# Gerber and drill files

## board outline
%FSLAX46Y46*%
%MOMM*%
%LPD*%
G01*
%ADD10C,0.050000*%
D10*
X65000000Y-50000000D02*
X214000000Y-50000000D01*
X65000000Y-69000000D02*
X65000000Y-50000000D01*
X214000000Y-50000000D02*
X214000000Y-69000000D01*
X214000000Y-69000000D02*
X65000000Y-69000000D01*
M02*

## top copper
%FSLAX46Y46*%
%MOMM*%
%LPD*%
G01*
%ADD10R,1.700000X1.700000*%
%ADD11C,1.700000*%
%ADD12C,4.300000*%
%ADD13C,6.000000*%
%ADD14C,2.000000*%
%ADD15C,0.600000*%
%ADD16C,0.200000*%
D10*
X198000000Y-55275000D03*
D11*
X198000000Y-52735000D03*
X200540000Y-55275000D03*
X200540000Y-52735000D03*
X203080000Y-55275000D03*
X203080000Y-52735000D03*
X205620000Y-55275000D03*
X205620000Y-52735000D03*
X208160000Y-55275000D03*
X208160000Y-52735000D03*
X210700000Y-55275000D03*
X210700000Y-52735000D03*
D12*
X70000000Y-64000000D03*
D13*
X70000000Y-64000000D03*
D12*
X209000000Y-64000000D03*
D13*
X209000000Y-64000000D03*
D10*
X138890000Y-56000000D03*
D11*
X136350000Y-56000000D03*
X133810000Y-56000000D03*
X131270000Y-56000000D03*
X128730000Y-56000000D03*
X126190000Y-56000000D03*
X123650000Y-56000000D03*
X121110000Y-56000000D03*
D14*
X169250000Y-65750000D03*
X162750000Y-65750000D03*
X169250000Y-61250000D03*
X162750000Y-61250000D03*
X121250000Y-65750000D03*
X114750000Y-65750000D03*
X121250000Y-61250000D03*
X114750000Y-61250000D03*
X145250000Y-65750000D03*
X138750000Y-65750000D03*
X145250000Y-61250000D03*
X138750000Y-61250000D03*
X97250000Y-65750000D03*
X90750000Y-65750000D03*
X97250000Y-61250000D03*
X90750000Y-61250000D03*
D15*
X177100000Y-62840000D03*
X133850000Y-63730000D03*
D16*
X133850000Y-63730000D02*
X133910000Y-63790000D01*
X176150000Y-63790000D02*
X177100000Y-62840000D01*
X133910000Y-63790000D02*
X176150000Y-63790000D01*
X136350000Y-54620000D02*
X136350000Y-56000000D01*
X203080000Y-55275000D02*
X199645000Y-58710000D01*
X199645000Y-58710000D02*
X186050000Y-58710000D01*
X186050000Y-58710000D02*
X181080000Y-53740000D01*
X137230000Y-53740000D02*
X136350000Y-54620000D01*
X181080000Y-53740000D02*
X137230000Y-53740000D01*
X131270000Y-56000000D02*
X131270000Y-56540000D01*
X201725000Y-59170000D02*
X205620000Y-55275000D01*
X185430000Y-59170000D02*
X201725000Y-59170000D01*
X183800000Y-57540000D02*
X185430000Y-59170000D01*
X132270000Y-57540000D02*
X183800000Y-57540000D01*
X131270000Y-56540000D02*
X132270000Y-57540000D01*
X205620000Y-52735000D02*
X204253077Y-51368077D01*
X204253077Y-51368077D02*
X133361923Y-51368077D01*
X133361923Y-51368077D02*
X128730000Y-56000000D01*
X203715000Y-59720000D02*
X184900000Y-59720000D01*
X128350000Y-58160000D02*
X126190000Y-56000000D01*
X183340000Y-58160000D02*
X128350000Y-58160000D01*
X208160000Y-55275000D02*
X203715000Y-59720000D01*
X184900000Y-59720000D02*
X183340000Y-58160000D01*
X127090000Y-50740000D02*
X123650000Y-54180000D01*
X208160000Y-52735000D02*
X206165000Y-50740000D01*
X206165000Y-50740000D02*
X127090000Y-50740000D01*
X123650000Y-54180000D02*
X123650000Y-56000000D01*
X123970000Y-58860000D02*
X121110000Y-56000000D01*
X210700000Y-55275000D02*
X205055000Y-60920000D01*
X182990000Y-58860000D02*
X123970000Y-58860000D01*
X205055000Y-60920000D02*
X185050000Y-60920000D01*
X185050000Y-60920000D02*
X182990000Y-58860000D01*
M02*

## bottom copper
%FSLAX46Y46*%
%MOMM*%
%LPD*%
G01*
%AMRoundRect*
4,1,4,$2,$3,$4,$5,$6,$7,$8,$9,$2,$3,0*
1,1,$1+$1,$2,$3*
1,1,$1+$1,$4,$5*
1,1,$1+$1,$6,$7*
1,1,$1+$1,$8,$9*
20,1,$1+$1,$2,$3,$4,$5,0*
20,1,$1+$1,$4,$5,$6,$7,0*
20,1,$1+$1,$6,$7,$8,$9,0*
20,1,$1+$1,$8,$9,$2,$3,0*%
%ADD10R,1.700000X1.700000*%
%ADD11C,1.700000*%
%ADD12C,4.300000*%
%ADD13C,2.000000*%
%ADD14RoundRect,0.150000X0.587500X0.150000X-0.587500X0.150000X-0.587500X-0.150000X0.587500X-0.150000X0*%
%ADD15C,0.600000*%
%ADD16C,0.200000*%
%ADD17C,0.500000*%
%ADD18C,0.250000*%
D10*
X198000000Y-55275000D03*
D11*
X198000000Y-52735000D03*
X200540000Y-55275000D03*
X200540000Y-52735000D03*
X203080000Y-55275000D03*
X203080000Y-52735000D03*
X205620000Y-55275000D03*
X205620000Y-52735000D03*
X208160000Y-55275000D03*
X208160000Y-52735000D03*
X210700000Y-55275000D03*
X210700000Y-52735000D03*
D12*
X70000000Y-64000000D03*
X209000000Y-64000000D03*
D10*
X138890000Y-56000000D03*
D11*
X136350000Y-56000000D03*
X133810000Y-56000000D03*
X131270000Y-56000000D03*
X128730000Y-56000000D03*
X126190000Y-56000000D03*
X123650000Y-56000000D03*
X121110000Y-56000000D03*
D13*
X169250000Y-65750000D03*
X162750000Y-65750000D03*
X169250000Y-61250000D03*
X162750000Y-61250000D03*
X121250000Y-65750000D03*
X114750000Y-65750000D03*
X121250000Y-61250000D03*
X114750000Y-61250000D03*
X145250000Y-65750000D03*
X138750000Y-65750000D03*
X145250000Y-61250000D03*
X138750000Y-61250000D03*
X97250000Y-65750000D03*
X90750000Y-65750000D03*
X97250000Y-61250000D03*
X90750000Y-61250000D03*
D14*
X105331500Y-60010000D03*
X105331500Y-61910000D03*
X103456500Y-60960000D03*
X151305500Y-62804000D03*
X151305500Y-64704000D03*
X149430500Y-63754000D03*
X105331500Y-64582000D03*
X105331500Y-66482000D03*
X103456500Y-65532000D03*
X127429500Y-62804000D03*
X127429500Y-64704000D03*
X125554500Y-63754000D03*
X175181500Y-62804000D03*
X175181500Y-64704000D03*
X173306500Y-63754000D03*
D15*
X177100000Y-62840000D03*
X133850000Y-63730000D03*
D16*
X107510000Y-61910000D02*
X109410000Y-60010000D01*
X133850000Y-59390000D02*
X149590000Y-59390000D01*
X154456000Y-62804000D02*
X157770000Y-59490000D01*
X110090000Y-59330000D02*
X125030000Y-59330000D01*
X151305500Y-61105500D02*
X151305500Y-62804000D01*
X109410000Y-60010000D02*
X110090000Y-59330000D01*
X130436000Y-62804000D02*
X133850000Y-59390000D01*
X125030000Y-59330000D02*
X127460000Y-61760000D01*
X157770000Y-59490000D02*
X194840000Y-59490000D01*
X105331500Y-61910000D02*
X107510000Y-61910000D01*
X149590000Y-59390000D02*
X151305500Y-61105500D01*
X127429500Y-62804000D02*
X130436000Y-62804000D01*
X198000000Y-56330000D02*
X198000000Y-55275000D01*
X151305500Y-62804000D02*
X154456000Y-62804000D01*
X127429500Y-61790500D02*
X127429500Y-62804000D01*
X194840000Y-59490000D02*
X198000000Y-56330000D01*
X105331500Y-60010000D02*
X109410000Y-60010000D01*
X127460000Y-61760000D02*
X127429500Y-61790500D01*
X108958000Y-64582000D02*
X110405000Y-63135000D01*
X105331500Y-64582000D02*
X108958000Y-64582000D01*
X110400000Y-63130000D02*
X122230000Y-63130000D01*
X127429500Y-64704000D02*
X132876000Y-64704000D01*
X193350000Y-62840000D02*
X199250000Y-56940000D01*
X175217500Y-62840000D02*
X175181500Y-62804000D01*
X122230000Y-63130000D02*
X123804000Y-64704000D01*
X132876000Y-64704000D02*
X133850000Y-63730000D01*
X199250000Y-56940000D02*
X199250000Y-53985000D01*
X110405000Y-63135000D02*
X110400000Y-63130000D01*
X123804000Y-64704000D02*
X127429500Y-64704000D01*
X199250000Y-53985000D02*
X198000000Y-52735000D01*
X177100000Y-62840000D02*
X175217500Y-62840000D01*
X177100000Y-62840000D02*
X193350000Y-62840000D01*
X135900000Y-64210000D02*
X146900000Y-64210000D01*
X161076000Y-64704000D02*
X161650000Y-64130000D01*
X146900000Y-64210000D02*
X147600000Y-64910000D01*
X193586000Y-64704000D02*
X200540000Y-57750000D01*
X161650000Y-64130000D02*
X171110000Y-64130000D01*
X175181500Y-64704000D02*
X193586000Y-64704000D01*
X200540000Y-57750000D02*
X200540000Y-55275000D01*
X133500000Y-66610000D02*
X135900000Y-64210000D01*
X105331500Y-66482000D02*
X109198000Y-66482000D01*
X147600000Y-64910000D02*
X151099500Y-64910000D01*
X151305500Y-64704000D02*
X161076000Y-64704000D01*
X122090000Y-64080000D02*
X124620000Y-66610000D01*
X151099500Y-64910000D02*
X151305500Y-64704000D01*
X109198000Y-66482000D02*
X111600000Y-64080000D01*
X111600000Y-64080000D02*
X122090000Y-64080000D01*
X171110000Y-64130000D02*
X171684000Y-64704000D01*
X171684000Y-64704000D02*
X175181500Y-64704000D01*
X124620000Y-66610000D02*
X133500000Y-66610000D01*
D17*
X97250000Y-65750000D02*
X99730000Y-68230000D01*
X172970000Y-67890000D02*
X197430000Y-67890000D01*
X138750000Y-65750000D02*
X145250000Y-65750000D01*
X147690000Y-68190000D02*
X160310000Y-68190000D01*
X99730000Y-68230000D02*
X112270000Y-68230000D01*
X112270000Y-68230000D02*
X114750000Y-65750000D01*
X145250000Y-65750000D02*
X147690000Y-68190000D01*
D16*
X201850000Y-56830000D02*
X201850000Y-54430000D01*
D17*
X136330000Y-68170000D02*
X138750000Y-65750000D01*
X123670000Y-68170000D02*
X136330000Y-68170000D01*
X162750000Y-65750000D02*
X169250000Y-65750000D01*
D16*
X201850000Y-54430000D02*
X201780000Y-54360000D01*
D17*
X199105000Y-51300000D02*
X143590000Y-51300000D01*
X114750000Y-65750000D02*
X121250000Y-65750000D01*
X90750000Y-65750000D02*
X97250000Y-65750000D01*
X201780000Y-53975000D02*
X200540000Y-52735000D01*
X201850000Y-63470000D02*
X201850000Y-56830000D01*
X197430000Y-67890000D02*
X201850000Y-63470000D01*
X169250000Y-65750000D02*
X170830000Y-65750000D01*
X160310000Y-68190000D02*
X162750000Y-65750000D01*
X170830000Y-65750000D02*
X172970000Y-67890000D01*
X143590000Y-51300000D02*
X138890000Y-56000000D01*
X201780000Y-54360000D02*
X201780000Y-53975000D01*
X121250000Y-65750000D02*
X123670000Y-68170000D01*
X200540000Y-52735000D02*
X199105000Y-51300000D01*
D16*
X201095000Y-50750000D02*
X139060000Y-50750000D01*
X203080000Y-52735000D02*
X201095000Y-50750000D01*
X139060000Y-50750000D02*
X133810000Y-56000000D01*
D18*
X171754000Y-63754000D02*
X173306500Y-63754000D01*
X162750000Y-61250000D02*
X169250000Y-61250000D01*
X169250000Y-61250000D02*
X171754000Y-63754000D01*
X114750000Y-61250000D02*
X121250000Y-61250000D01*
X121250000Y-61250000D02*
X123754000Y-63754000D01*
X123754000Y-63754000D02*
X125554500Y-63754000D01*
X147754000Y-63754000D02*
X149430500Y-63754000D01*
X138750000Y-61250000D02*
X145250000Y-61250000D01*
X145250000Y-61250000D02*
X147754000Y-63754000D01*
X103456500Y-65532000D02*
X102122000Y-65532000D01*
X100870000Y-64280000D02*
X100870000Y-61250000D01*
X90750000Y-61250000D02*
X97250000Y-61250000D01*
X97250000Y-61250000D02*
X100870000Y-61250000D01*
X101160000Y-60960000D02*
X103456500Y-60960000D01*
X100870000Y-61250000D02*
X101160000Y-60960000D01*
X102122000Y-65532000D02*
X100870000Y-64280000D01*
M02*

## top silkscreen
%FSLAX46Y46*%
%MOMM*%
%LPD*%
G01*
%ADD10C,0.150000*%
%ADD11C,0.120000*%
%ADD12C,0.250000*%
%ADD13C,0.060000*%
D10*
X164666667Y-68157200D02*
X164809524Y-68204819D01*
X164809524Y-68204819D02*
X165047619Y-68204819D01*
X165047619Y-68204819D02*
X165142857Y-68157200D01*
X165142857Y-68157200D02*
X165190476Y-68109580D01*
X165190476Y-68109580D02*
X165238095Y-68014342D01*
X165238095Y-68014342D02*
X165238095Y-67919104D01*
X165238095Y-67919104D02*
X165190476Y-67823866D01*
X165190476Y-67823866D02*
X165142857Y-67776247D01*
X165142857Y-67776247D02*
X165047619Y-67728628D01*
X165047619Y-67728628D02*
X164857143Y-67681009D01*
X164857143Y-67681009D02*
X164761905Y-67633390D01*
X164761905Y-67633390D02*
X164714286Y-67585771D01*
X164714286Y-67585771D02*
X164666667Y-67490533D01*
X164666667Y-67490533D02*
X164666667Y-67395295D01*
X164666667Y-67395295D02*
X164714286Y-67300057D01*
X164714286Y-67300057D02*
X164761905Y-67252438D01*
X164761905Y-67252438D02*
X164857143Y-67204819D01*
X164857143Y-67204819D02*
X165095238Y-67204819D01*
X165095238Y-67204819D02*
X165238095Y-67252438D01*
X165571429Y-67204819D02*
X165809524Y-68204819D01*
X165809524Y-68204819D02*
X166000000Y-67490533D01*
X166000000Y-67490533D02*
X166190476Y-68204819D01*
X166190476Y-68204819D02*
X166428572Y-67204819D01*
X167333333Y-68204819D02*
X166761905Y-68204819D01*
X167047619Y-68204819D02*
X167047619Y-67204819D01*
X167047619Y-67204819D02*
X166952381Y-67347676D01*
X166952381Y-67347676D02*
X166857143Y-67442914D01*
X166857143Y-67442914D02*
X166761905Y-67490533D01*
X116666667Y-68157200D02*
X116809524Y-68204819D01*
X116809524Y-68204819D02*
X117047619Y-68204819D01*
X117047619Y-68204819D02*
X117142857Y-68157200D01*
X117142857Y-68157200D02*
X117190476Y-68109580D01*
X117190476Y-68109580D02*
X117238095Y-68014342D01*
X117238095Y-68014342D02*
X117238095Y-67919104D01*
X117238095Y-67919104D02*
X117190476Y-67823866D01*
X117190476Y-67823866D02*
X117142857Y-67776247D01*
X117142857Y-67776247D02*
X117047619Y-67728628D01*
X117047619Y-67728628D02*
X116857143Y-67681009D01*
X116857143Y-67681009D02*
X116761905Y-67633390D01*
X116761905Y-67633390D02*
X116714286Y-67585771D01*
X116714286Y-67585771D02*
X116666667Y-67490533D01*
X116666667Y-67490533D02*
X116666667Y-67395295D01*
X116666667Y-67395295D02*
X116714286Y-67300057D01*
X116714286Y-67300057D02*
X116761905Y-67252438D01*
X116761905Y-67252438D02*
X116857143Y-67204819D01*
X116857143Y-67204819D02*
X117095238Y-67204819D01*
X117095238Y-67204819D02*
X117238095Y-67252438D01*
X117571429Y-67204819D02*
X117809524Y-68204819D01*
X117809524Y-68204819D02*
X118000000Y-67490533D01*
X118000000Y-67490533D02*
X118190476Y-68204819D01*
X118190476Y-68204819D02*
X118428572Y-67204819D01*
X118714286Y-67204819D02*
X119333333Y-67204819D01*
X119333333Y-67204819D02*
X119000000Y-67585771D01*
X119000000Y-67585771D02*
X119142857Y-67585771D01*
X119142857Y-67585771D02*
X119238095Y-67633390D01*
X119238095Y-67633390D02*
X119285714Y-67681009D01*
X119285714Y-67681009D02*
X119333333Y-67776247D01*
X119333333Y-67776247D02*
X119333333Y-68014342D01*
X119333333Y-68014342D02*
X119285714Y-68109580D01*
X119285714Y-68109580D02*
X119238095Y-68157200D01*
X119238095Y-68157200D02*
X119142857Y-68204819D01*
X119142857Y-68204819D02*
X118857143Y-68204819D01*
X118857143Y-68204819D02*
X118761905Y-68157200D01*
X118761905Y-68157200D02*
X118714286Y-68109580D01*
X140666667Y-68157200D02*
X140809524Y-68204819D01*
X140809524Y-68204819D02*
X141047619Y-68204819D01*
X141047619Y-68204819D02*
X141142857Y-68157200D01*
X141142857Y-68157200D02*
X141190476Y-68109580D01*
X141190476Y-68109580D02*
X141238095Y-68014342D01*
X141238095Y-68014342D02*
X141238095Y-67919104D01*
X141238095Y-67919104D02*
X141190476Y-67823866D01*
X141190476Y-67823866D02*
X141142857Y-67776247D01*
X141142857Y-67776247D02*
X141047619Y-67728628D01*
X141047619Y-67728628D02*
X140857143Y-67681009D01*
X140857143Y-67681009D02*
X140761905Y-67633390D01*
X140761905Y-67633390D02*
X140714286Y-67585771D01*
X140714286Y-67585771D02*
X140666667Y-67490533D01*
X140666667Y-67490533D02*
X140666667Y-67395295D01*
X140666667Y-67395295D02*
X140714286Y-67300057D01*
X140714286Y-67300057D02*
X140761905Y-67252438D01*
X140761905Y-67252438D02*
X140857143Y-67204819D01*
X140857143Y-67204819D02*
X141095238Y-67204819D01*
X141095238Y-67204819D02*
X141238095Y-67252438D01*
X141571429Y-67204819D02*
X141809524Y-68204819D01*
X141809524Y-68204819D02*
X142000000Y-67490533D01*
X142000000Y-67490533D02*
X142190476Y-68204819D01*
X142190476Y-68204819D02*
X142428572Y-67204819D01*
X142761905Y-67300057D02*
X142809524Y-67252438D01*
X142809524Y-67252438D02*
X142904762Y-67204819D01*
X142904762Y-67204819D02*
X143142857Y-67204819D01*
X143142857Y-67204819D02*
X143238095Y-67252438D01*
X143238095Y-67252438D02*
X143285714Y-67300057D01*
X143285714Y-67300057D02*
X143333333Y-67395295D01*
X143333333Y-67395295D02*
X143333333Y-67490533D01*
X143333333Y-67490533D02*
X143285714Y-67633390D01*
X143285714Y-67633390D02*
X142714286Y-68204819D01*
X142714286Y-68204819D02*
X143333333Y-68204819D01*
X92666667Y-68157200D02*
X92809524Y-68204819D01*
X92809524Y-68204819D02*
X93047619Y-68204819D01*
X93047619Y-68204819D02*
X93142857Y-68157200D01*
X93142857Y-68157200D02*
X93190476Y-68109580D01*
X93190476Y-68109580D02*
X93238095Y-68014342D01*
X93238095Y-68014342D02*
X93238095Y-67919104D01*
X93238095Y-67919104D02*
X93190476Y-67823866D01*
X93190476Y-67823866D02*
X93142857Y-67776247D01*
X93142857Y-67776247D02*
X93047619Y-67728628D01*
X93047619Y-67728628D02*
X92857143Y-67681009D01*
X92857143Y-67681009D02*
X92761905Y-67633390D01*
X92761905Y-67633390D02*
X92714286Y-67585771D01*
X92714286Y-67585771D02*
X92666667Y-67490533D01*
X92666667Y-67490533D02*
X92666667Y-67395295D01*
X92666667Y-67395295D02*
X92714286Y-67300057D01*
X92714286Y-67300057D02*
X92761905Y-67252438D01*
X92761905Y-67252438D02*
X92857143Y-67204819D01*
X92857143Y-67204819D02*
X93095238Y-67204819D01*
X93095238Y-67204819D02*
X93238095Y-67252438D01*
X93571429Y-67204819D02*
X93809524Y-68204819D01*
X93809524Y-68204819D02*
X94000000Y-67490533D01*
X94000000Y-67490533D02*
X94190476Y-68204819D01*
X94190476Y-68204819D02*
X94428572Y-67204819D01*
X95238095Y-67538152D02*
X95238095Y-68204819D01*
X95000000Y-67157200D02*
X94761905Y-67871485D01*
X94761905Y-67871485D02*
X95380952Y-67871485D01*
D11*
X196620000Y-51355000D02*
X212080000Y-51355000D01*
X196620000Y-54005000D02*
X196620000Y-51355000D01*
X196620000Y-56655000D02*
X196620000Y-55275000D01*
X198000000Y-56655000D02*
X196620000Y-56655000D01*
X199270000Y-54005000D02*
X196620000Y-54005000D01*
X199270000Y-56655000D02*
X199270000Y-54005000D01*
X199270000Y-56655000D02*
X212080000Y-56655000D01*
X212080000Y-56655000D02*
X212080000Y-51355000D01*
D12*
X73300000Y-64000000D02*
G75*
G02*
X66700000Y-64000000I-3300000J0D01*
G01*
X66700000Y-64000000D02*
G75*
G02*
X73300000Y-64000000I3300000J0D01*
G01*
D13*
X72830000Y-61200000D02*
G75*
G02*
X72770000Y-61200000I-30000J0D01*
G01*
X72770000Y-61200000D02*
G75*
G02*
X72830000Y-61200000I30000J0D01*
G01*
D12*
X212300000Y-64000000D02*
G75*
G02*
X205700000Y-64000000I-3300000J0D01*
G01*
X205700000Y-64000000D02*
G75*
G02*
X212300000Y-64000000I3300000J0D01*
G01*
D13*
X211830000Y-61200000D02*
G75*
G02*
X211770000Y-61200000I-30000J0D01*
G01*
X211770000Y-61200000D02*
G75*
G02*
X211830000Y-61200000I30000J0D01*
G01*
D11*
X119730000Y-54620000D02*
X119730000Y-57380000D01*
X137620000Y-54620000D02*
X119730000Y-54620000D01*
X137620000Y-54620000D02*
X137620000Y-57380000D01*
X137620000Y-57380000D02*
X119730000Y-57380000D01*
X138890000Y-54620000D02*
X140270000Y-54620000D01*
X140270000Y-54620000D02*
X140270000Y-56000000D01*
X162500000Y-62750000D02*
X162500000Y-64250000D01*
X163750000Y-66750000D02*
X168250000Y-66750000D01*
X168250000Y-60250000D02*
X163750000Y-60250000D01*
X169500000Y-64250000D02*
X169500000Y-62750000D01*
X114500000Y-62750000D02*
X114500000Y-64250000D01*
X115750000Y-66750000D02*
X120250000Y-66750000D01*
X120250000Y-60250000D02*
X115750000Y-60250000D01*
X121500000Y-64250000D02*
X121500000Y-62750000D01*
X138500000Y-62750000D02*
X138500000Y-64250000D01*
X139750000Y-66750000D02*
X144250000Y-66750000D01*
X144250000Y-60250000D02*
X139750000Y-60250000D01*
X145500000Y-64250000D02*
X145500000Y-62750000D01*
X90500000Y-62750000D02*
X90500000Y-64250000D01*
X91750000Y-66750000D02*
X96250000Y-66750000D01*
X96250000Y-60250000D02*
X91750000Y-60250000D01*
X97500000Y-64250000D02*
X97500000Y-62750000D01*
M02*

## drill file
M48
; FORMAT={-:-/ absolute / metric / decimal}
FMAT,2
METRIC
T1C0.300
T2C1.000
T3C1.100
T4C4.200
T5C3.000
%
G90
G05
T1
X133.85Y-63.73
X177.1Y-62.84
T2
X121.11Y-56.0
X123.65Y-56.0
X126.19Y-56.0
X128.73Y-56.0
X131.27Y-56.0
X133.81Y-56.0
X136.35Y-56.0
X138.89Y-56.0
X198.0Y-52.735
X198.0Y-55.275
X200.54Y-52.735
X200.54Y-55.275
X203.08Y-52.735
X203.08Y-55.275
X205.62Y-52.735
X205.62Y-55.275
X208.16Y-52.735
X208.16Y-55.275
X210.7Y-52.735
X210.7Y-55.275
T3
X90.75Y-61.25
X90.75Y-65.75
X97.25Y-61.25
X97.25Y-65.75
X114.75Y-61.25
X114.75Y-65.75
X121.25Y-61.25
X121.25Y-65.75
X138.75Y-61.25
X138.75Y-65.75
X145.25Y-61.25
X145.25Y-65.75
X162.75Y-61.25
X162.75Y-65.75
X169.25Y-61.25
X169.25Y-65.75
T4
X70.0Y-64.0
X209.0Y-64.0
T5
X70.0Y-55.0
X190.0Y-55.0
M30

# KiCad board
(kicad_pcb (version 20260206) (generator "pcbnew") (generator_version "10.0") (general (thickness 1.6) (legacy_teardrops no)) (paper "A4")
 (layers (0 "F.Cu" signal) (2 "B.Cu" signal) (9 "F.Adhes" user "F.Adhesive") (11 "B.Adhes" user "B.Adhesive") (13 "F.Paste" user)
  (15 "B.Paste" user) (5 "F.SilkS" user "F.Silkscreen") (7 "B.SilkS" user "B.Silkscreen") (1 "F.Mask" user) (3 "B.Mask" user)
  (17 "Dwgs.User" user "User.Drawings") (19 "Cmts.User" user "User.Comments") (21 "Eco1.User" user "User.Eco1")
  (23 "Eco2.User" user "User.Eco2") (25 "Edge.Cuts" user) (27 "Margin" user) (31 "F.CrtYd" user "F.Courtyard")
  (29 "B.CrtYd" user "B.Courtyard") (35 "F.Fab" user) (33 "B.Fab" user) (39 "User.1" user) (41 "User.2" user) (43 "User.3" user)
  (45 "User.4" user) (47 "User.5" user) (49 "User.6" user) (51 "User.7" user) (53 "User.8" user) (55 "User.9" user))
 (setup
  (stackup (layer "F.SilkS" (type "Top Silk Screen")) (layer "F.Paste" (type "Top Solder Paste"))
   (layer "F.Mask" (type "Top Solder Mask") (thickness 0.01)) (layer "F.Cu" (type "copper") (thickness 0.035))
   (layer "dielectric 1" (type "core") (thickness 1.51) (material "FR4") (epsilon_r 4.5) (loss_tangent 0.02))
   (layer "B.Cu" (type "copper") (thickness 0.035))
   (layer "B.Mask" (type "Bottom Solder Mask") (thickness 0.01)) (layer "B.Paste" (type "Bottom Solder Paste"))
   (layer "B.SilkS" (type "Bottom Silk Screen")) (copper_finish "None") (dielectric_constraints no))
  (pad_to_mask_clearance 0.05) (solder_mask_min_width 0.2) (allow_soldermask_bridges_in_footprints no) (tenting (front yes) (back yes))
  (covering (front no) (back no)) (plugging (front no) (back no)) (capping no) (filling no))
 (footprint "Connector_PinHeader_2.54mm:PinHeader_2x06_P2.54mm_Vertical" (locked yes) (layer "F.Cu") (at 198 55.275 90)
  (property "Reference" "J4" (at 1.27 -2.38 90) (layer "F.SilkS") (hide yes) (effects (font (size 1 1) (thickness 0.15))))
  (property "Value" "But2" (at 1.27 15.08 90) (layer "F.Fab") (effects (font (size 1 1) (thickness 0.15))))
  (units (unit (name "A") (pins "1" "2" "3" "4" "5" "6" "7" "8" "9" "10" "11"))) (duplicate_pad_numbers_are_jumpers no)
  (fp_line (start 3.92 -1.38) (end 3.92 14.08) (stroke (width 0.12) (type solid)) (layer "F.SilkS"))
  (fp_line (start 1.27 -1.38) (end 3.92 -1.38) (stroke (width 0.12) (type solid)) (layer "F.SilkS"))
  (fp_line (start -1.38 -1.38) (end 0 -1.38) (stroke (width 0.12) (type solid)) (layer "F.SilkS"))
  (fp_line (start -1.38 0) (end -1.38 -1.38) (stroke (width 0.12) (type solid)) (layer "F.SilkS"))
  (fp_line (start 1.27 1.27) (end 1.27 -1.38) (stroke (width 0.12) (type solid)) (layer "F.SilkS"))
  (fp_line (start -1.38 1.27) (end 1.27 1.27) (stroke (width 0.12) (type solid)) (layer "F.SilkS"))
  (fp_line (start -1.38 1.27) (end -1.38 14.08) (stroke (width 0.12) (type solid)) (layer "F.SilkS"))
  (fp_line (start -1.38 14.08) (end 3.92 14.08) (stroke (width 0.12) (type solid)) (layer "F.SilkS"))
  (pad "1" thru_hole rect (at 0 0 90) (size 1.7 1.7) (drill 1) (layers "*.Cu" "*.Mask") (remove_unused_layers no) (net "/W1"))
  (pad "2" thru_hole circle (at 2.54 0 90) (size 1.7 1.7) (drill 1) (layers "*.Cu" "*.Mask") (remove_unused_layers no) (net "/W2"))
  (pad "3" thru_hole circle (at 0 2.54 90) (size 1.7 1.7) (drill 1) (layers "*.Cu" "*.Mask") (remove_unused_layers no) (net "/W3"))
  (pad "4" thru_hole circle (at 2.54 2.54 90) (size 1.7 1.7) (drill 1) (layers "*.Cu" "*.Mask") (remove_unused_layers no) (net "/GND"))
  (pad "5" thru_hole circle (at 0 5.08 90) (size 1.7 1.7) (drill 1) (layers "*.Cu" "*.Mask") (remove_unused_layers no)
   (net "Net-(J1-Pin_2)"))
  (pad "6" thru_hole circle (at 2.54 5.08 90) (size 1.7 1.7) (drill 1) (layers "*.Cu" "*.Mask") (remove_unused_layers no)
   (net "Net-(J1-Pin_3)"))
  (pad "7" thru_hole circle (at 0 7.62 90) (size 1.7 1.7) (drill 1) (layers "*.Cu" "*.Mask") (remove_unused_layers no)
   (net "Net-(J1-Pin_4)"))
  (pad "8" thru_hole circle (at 2.54 7.62 90) (size 1.7 1.7) (drill 1) (layers "*.Cu" "*.Mask") (remove_unused_layers no)
   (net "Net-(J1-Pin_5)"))
  (pad "9" thru_hole circle (at 0 10.16 90) (size 1.7 1.7) (drill 1) (layers "*.Cu" "*.Mask") (remove_unused_layers no)
   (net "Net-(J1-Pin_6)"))
  (pad "10" thru_hole circle (at 2.54 10.16 90) (size 1.7 1.7) (drill 1) (layers "*.Cu" "*.Mask") (remove_unused_layers no)
   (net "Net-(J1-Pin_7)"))
  (pad "11" thru_hole circle (at 0 12.7 90) (size 1.7 1.7) (drill 1) (layers "*.Cu" "*.Mask") (remove_unused_layers no)
   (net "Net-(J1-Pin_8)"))
  (pad "12" thru_hole circle (at 2.54 12.7 90) (size 1.7 1.7) (drill 1) (layers "*.Cu" "*.Mask") (remove_unused_layers no)))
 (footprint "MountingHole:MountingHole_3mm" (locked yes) (layer "F.Cu") (at 70 55)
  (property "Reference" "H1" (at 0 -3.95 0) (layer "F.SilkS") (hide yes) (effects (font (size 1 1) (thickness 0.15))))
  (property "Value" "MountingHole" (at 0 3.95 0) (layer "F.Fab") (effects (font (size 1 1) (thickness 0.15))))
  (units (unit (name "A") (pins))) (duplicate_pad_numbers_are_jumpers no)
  (pad "" np_thru_hole circle (at 0 0) (size 3 3) (drill 3) (layers "*.Cu" "*.Mask")))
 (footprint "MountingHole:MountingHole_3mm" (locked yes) (layer "F.Cu") (at 190 55)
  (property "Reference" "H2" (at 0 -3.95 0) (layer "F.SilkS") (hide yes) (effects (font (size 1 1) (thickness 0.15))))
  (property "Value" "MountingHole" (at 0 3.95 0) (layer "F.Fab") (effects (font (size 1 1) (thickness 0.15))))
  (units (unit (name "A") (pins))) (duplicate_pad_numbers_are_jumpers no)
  (pad "" np_thru_hole circle (at 0 0) (size 3 3) (drill 3) (layers "*.Cu" "*.Mask")))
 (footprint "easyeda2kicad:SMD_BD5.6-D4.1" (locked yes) (layer "F.Cu") (at 70 64)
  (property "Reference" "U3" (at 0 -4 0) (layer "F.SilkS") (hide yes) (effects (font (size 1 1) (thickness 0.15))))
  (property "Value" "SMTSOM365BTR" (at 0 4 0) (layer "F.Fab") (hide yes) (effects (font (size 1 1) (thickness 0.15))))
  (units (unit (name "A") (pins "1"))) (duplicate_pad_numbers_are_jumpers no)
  (fp_circle (center 0 0) (end 3.3 0) (stroke (width 0.25) (type solid)) (fill no) (layer "F.SilkS"))
  (fp_circle (center 2.8 -2.8) (end 2.83 -2.8) (stroke (width 0.06) (type solid)) (fill no) (layer "F.SilkS"))
  (pad "1" thru_hole circle (at 0 0) (size 4.3 4.3) (drill 4.199992) (layers "*.Cu" "*.Mask") (remove_unused_layers no)
   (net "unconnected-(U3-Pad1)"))
  (pad "1" smd circle (at 0 0) (size 6 6) (layers "F.Cu" "F.Mask" "F.Paste") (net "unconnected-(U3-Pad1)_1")))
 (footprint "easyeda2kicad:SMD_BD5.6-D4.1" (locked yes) (layer "F.Cu") (at 209 64)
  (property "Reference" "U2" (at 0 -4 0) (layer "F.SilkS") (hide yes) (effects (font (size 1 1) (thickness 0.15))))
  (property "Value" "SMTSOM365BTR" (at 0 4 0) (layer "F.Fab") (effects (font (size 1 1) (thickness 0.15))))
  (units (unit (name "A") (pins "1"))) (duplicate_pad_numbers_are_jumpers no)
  (fp_circle (center 0 0) (end 3.3 0) (stroke (width 0.25) (type solid)) (fill no) (layer "F.SilkS"))
  (fp_circle (center 2.8 -2.8) (end 2.83 -2.8) (stroke (width 0.06) (type solid)) (fill no) (layer "F.SilkS"))
  (pad "1" thru_hole circle (at 0 0) (size 4.3 4.3) (drill 4.199992) (layers "*.Cu" "*.Mask") (remove_unused_layers no)
   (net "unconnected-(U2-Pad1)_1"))
  (pad "1" smd circle (at 0 0) (size 6 6) (layers "F.Cu" "F.Mask" "F.Paste") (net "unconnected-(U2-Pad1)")))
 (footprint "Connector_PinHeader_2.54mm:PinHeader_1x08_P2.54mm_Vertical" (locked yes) (layer "F.Cu") (at 138.89 56 -90)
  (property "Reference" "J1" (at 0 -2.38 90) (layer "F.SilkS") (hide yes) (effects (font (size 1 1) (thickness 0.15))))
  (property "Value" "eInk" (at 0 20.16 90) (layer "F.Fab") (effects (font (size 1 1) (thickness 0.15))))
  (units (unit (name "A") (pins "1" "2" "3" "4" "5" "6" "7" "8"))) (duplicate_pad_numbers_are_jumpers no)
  (fp_line (start -1.38 19.16) (end 1.38 19.16) (stroke (width 0.12) (type solid)) (layer "F.SilkS"))
  (fp_line (start -1.38 1.27) (end -1.38 19.16) (stroke (width 0.12) (type solid)) (layer "F.SilkS"))
  (fp_line (start -1.38 1.27) (end 1.38 1.27) (stroke (width 0.12) (type solid)) (layer "F.SilkS"))
  (fp_line (start 1.38 1.27) (end 1.38 19.16) (stroke (width 0.12) (type solid)) (layer "F.SilkS"))
  (fp_line (start -1.38 0) (end -1.38 -1.38) (stroke (width 0.12) (type solid)) (layer "F.SilkS"))
  (fp_line (start -1.38 -1.38) (end 0 -1.38) (stroke (width 0.12) (type solid)) (layer "F.SilkS"))
  (pad "1" thru_hole rect (at 0 0 270) (size 1.7 1.7) (drill 1) (layers "*.Cu" "*.Mask") (remove_unused_layers no) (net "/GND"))
  (pad "2" thru_hole circle (at 0 2.54 270) (size 1.7 1.7) (drill 1) (layers "*.Cu" "*.Mask") (remove_unused_layers no)
   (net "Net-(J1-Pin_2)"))
  (pad "3" thru_hole circle (at 0 5.08 270) (size 1.7 1.7) (drill 1) (layers "*.Cu" "*.Mask") (remove_unused_layers no)
   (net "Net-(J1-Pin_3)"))
  (pad "4" thru_hole circle (at 0 7.62 270) (size 1.7 1.7) (drill 1) (layers "*.Cu" "*.Mask") (remove_unused_layers no)
   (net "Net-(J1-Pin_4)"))
  (pad "5" thru_hole circle (at 0 10.16 270) (size 1.7 1.7) (drill 1) (layers "*.Cu" "*.Mask") (remove_unused_layers no)
   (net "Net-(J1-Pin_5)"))
  (pad "6" thru_hole circle (at 0 12.7 270) (size 1.7 1.7) (drill 1) (layers "*.Cu" "*.Mask") (remove_unused_layers no)
   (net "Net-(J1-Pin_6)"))
  (pad "7" thru_hole circle (at 0 15.24 270) (size 1.7 1.7) (drill 1) (layers "*.Cu" "*.Mask") (remove_unused_layers no)
   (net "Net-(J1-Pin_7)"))
  (pad "8" thru_hole circle (at 0 17.78 270) (size 1.7 1.7) (drill 1) (layers "*.Cu" "*.Mask") (remove_unused_layers no)
   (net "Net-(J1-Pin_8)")))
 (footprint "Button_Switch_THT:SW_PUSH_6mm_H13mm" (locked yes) (layer "F.Cu") (at 169.25 65.75 180)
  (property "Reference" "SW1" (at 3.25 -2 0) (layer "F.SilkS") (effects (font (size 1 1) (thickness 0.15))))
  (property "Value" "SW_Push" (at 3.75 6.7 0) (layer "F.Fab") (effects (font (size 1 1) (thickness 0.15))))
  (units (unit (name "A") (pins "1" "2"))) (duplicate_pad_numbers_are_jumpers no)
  (fp_line (start 6.75 3) (end 6.75 1.5) (stroke (width 0.12) (type solid)) (layer "F.SilkS"))
  (fp_line (start 5.5 -1) (end 1 -1) (stroke (width 0.12) (type solid)) (layer "F.SilkS"))
  (fp_line (start 1 5.5) (end 5.5 5.5) (stroke (width 0.12) (type solid)) (layer "F.SilkS"))
  (fp_line (start -0.25 1.5) (end -0.25 3) (stroke (width 0.12) (type solid)) (layer "F.SilkS"))
  (pad "1" thru_hole circle (at 0 0 270) (size 2 2) (drill 1.1) (layers "*.Cu" "*.Mask") (remove_unused_layers no) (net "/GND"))
  (pad "1" thru_hole circle (at 6.5 0 270) (size 2 2) (drill 1.1) (layers "*.Cu" "*.Mask") (remove_unused_layers no) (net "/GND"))
  (pad "2" thru_hole circle (at 0 4.5 270) (size 2 2) (drill 1.1) (layers "*.Cu" "*.Mask") (remove_unused_layers no) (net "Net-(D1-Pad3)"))
  (pad "2" thru_hole circle (at 6.5 4.5 270) (size 2 2) (drill 1.1) (layers "*.Cu" "*.Mask") (remove_unused_layers no) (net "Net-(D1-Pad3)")))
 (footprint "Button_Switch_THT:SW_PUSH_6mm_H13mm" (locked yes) (layer "F.Cu") (at 121.25 65.75 180)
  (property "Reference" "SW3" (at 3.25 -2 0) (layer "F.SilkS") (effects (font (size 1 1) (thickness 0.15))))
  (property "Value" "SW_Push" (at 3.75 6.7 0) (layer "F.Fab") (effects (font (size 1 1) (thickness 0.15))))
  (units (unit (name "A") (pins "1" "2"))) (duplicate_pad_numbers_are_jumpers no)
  (fp_line (start 6.75 3) (end 6.75 1.5) (stroke (width 0.12) (type solid)) (layer "F.SilkS"))
  (fp_line (start 5.5 -1) (end 1 -1) (stroke (width 0.12) (type solid)) (layer "F.SilkS"))
  (fp_line (start 1 5.5) (end 5.5 5.5) (stroke (width 0.12) (type solid)) (layer "F.SilkS"))
  (fp_line (start -0.25 1.5) (end -0.25 3) (stroke (width 0.12) (type solid)) (layer "F.SilkS"))
  (pad "1" thru_hole circle (at 0 0 270) (size 2 2) (drill 1.1) (layers "*.Cu" "*.Mask") (remove_unused_layers no) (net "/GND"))
  (pad "1" thru_hole circle (at 6.5 0 270) (size 2 2) (drill 1.1) (layers "*.Cu" "*.Mask") (remove_unused_layers no) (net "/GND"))
  (pad "2" thru_hole circle (at 0 4.5 270) (size 2 2) (drill 1.1) (layers "*.Cu" "*.Mask") (remove_unused_layers no) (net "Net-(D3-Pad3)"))
  (pad "2" thru_hole circle (at 6.5 4.5 270) (size 2 2) (drill 1.1) (layers "*.Cu" "*.Mask") (remove_unused_layers no) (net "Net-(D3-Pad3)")))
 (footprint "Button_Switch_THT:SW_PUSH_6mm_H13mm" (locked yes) (layer "F.Cu") (at 145.25 65.75 180)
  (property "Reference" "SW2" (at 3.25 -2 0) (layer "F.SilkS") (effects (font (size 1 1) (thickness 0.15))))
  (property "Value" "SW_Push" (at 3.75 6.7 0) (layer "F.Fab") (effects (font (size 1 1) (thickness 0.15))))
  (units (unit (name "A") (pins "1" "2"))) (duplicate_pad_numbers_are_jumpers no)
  (fp_line (start 6.75 3) (end 6.75 1.5) (stroke (width 0.12) (type solid)) (layer "F.SilkS"))
  (fp_line (start 5.5 -1) (end 1 -1) (stroke (width 0.12) (type solid)) (layer "F.SilkS"))
  (fp_line (start 1 5.5) (end 5.5 5.5) (stroke (width 0.12) (type solid)) (layer "F.SilkS"))
  (fp_line (start -0.25 1.5) (end -0.25 3) (stroke (width 0.12) (type solid)) (layer "F.SilkS"))
  (pad "1" thru_hole circle (at 0 0 270) (size 2 2) (drill 1.1) (layers "*.Cu" "*.Mask") (remove_unused_layers no) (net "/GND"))
  (pad "1" thru_hole circle (at 6.5 0 270) (size 2 2) (drill 1.1) (layers "*.Cu" "*.Mask") (remove_unused_layers no) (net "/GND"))
  (pad "2" thru_hole circle (at 0 4.5 270) (size 2 2) (drill 1.1) (layers "*.Cu" "*.Mask") (remove_unused_layers no) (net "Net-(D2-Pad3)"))
  (pad "2" thru_hole circle (at 6.5 4.5 270) (size 2 2) (drill 1.1) (layers "*.Cu" "*.Mask") (remove_unused_layers no) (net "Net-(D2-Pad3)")))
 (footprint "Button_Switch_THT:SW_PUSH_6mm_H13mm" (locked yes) (layer "F.Cu") (at 97.25 65.75 180)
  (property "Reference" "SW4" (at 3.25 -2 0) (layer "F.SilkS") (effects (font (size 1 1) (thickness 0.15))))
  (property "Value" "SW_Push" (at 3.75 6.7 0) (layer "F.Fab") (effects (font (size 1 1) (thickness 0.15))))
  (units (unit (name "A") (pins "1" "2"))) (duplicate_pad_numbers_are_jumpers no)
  (fp_line (start 6.75 3) (end 6.75 1.5) (stroke (width 0.12) (type solid)) (layer "F.SilkS"))
  (fp_line (start 5.5 -1) (end 1 -1) (stroke (width 0.12) (type solid)) (layer "F.SilkS"))
  (fp_line (start 1 5.5) (end 5.5 5.5) (stroke (width 0.12) (type solid)) (layer "F.SilkS"))
  (fp_line (start -0.25 1.5) (end -0.25 3) (stroke (width 0.12) (type solid)) (layer "F.SilkS"))
  (pad "1" thru_hole circle (at 0 0 270) (size 2 2) (drill 1.1) (layers "*.Cu" "*.Mask") (remove_unused_layers no) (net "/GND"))
  (pad "1" thru_hole circle (at 6.5 0 270) (size 2 2) (drill 1.1) (layers "*.Cu" "*.Mask") (remove_unused_layers no) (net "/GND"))
  (pad "2" thru_hole circle (at 0 4.5 270) (size 2 2) (drill 1.1) (layers "*.Cu" "*.Mask") (remove_unused_layers no) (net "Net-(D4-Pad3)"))
  (pad "2" thru_hole circle (at 6.5 4.5 270) (size 2 2) (drill 1.1) (layers "*.Cu" "*.Mask") (remove_unused_layers no) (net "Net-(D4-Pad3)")))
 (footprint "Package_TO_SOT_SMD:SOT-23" (layer "B.Cu") (at 104.394 60.96 180)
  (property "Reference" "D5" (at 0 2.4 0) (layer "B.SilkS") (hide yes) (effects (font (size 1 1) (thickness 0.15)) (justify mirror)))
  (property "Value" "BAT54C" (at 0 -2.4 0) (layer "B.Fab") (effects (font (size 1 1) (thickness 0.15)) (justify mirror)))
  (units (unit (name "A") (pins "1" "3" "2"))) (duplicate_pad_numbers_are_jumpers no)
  (pad "1" smd roundrect (at -0.9375 0.95 180) (size 1.475 0.6) (layers "B.Cu" "B.Mask" "B.Paste") (roundrect_rratio 0.25) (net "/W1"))
  (pad "2" smd roundrect (at -0.9375 -0.95 180) (size 1.475 0.6) (layers "B.Cu" "B.Mask" "B.Paste") (roundrect_rratio 0.25) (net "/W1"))
  (pad "3" smd roundrect (at 0.9375 0 180) (size 1.475 0.6) (layers "B.Cu" "B.Mask" "B.Paste") (roundrect_rratio 0.25) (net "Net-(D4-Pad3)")))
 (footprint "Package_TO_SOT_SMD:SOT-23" (layer "B.Cu") (at 150.368 63.754 180)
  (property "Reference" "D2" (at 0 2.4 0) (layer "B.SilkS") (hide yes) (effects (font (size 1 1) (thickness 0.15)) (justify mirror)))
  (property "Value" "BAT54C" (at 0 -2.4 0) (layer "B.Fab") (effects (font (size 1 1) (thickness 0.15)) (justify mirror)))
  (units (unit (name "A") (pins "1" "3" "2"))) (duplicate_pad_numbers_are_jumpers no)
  (pad "1" smd roundrect (at -0.9375 0.95 180) (size 1.475 0.6) (layers "B.Cu" "B.Mask" "B.Paste") (roundrect_rratio 0.25) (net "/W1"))
  (pad "2" smd roundrect (at -0.9375 -0.95 180) (size 1.475 0.6) (layers "B.Cu" "B.Mask" "B.Paste") (roundrect_rratio 0.25) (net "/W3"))
  (pad "3" smd roundrect (at 0.9375 0 180) (size 1.475 0.6) (layers "B.Cu" "B.Mask" "B.Paste") (roundrect_rratio 0.25) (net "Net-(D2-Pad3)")))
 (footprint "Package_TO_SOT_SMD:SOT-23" (layer "B.Cu") (at 104.394 65.532 180)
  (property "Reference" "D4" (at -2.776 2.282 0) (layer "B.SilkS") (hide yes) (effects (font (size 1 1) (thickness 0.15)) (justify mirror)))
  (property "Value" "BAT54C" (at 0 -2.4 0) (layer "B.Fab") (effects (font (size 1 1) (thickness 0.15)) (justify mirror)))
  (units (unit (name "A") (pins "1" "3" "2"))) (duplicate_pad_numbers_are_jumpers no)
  (pad "1" smd roundrect (at -0.9375 0.95 180) (size 1.475 0.6) (layers "B.Cu" "B.Mask" "B.Paste") (roundrect_rratio 0.25) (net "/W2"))
  (pad "2" smd roundrect (at -0.9375 -0.95 180) (size 1.475 0.6) (layers "B.Cu" "B.Mask" "B.Paste") (roundrect_rratio 0.25) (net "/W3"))
  (pad "3" smd roundrect (at 0.9375 0 180) (size 1.475 0.6) (layers "B.Cu" "B.Mask" "B.Paste") (roundrect_rratio 0.25) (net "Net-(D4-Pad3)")))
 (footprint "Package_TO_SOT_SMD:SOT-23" (layer "B.Cu") (at 126.492 63.754 180)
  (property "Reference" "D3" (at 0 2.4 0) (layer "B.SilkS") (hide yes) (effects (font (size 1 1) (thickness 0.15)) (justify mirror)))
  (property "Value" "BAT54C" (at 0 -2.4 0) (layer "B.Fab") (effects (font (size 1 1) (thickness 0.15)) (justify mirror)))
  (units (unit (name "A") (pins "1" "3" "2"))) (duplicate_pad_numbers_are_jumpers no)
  (pad "1" smd roundrect (at -0.9375 0.95 180) (size 1.475 0.6) (layers "B.Cu" "B.Mask" "B.Paste") (roundrect_rratio 0.25) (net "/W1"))
  (pad "2" smd roundrect (at -0.9375 -0.95 180) (size 1.475 0.6) (layers "B.Cu" "B.Mask" "B.Paste") (roundrect_rratio 0.25) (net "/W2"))
  (pad "3" smd roundrect (at 0.9375 0 180) (size 1.475 0.6) (layers "B.Cu" "B.Mask" "B.Paste") (roundrect_rratio 0.25) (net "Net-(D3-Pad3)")))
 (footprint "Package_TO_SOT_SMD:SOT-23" (layer "B.Cu") (at 174.244 63.754 180)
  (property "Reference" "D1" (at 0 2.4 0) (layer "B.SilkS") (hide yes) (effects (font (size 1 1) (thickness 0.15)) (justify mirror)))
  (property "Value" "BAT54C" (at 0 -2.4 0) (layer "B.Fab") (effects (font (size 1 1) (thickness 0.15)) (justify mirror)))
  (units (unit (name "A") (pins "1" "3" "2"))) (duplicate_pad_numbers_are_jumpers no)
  (pad "1" smd roundrect (at -0.9375 0.95 180) (size 1.475 0.6) (layers "B.Cu" "B.Mask" "B.Paste") (roundrect_rratio 0.25) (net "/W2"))
  (pad "2" smd roundrect (at -0.9375 -0.95 180) (size 1.475 0.6) (layers "B.Cu" "B.Mask" "B.Paste") (roundrect_rratio 0.25) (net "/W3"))
  (pad "3" smd roundrect (at 0.9375 0 180) (size 1.475 0.6) (layers "B.Cu" "B.Mask" "B.Paste") (roundrect_rratio 0.25) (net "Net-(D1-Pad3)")))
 (gr_line (start 65 50) (end 214 50) (stroke (width 0.05) (type default)) (layer "Edge.Cuts"))
 (gr_line (start 65 69) (end 65 50) (stroke (width 0.05) (type default)) (layer "Edge.Cuts"))
 (gr_line (start 214 50) (end 214 69) (stroke (width 0.05) (type default)) (layer "Edge.Cuts"))
 (gr_line (start 214 69) (end 65 69) (stroke (width 0.05) (type default)) (layer "Edge.Cuts"))
 (segment (start 107.51 61.91) (end 109.41 60.01) (width 0.2) (layer "B.Cu") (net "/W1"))
 (segment (start 133.85 59.39) (end 149.59 59.39) (width 0.2) (layer "B.Cu") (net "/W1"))
 (segment (start 154.456 62.804) (end 157.77 59.49) (width 0.2) (layer "B.Cu") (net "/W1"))
 (segment (start 110.09 59.33) (end 125.03 59.33) (width 0.2) (layer "B.Cu") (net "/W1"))
 (segment (start 151.3055 61.1055) (end 151.3055 62.804) (width 0.2) (layer "B.Cu") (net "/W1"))
 (segment (start 109.41 60.01) (end 110.09 59.33) (width 0.2) (layer "B.Cu") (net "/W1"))
 (segment (start 130.436 62.804) (end 133.85 59.39) (width 0.2) (layer "B.Cu") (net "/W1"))
 (segment (start 125.03 59.33) (end 127.46 61.76) (width 0.2) (layer "B.Cu") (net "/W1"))
 (segment (start 157.77 59.49) (end 194.84 59.49) (width 0.2) (layer "B.Cu") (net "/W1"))
 (segment (start 105.3315 61.91) (end 107.51 61.91) (width 0.2) (layer "B.Cu") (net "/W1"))
 (segment (start 149.59 59.39) (end 151.3055 61.1055) (width 0.2) (layer "B.Cu") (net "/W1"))
 (segment (start 127.4295 62.804) (end 130.436 62.804) (width 0.2) (layer "B.Cu") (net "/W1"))
 (segment (start 198 56.33) (end 198 55.275) (width 0.2) (layer "B.Cu") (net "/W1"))
 (segment (start 151.3055 62.804) (end 154.456 62.804) (width 0.2) (layer "B.Cu") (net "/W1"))
 (segment (start 127.4295 61.7905) (end 127.4295 62.804) (width 0.2) (layer "B.Cu") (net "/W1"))
 (segment (start 194.84 59.49) (end 198 56.33) (width 0.2) (layer "B.Cu") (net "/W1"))
 (segment (start 105.3315 60.01) (end 109.41 60.01) (width 0.2) (layer "B.Cu") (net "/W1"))
 (segment (start 127.46 61.76) (end 127.4295 61.7905) (width 0.2) (layer "B.Cu") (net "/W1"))
 (segment (start 133.85 63.73) (end 133.91 63.79) (width 0.2) (layer "F.Cu") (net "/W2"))
 (segment (start 176.15 63.79) (end 177.1 62.84) (width 0.2) (layer "F.Cu") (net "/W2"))
 (segment (start 133.91 63.79) (end 176.15 63.79) (width 0.2) (layer "F.Cu") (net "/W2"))
 (via (at 177.1 62.84) (size 0.6) (drill 0.3) (layers "F.Cu" "B.Cu") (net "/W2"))
 (via (at 133.85 63.73) (size 0.6) (drill 0.3) (layers "F.Cu" "B.Cu") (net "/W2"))
 (segment (start 108.958 64.582) (end 110.405 63.135) (width 0.2) (layer "B.Cu") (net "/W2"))
 (segment (start 105.3315 64.582) (end 108.958 64.582) (width 0.2) (layer "B.Cu") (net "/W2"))
 (segment (start 110.4 63.13) (end 122.23 63.13) (width 0.2) (layer "B.Cu") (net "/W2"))
 (segment (start 127.4295 64.704) (end 132.876 64.704) (width 0.2) (layer "B.Cu") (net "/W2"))
 (segment (start 193.35 62.84) (end 199.25 56.94) (width 0.2) (layer "B.Cu") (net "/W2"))
 (segment (start 175.2175 62.84) (end 175.1815 62.804) (width 0.2) (layer "B.Cu") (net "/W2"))
 (segment (start 122.23 63.13) (end 123.804 64.704) (width 0.2) (layer "B.Cu") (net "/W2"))
 (segment (start 132.876 64.704) (end 133.85 63.73) (width 0.2) (layer "B.Cu") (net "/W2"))
 (segment (start 199.25 56.94) (end 199.25 53.985) (width 0.2) (layer "B.Cu") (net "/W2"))
 (segment (start 110.405 63.135) (end 110.4 63.13) (width 0.2) (layer "B.Cu") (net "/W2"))
 (segment (start 123.804 64.704) (end 127.4295 64.704) (width 0.2) (layer "B.Cu") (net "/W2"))
 (segment (start 199.25 53.985) (end 198 52.735) (width 0.2) (layer "B.Cu") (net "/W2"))
 (segment (start 177.1 62.84) (end 175.2175 62.84) (width 0.2) (layer "B.Cu") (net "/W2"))
 (segment (start 177.1 62.84) (end 193.35 62.84) (width 0.2) (layer "B.Cu") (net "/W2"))
 (segment (start 135.9 64.21) (end 146.9 64.21) (width 0.2) (layer "B.Cu") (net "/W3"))
 (segment (start 161.076 64.704) (end 161.65 64.13) (width 0.2) (layer "B.Cu") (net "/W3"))
 (segment (start 146.9 64.21) (end 147.6 64.91) (width 0.2) (layer "B.Cu") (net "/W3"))
 (segment (start 193.586 64.704) (end 200.54 57.75) (width 0.2) (layer "B.Cu") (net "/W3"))
 (segment (start 161.65 64.13) (end 171.11 64.13) (width 0.2) (layer "B.Cu") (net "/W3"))
 (segment (start 175.1815 64.704) (end 193.586 64.704) (width 0.2) (layer "B.Cu") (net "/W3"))
 (segment (start 200.54 57.75) (end 200.54 55.275) (width 0.2) (layer "B.Cu") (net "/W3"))
 (segment (start 133.5 66.61) (end 135.9 64.21) (width 0.2) (layer "B.Cu") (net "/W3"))
 (segment (start 105.3315 66.482) (end 109.198 66.482) (width 0.2) (layer "B.Cu") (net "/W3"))
 (segment (start 147.6 64.91) (end 151.0995 64.91) (width 0.2) (layer "B.Cu") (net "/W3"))
 (segment (start 151.3055 64.704) (end 161.076 64.704) (width 0.2) (layer "B.Cu") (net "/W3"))
 (segment (start 122.09 64.08) (end 124.62 66.61) (width 0.2) (layer "B.Cu") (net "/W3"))
 (segment (start 151.0995 64.91) (end 151.3055 64.704) (width 0.2) (layer "B.Cu") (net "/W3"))
 (segment (start 109.198 66.482) (end 111.6 64.08) (width 0.2) (layer "B.Cu") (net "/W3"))
 (segment (start 111.6 64.08) (end 122.09 64.08) (width 0.2) (layer "B.Cu") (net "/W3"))
 (segment (start 171.11 64.13) (end 171.684 64.704) (width 0.2) (layer "B.Cu") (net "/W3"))
 (segment (start 171.684 64.704) (end 175.1815 64.704) (width 0.2) (layer "B.Cu") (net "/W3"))
 (segment (start 124.62 66.61) (end 133.5 66.61) (width 0.2) (layer "B.Cu") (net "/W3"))
 (segment (start 97.25 65.75) (end 99.73 68.23) (width 0.5) (layer "B.Cu") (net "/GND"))
 (segment (start 172.97 67.89) (end 197.43 67.89) (width 0.5) (layer "B.Cu") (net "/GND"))
 (segment (start 138.75 65.75) (end 145.25 65.75) (width 0.5) (layer "B.Cu") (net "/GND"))
 (segment (start 147.69 68.19) (end 160.31 68.19) (width 0.5) (layer "B.Cu") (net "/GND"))
 (segment (start 99.73 68.23) (end 112.27 68.23) (width 0.5) (layer "B.Cu") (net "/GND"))
 (segment (start 112.27 68.23) (end 114.75 65.75) (width 0.5) (layer "B.Cu") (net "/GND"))
 (segment (start 145.25 65.75) (end 147.69 68.19) (width 0.5) (layer "B.Cu") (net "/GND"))
 (segment (start 201.85 56.83) (end 201.85 54.43) (width 0.2) (layer "B.Cu") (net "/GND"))
 (segment (start 136.33 68.17) (end 138.75 65.75) (width 0.5) (layer "B.Cu") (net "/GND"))
 (segment (start 123.67 68.17) (end 136.33 68.17) (width 0.5) (layer "B.Cu") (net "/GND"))
 (segment (start 162.75 65.75) (end 169.25 65.75) (width 0.5) (layer "B.Cu") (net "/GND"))
 (segment (start 201.85 54.43) (end 201.78 54.36) (width 0.2) (layer "B.Cu") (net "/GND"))
 (segment (start 199.105 51.3) (end 143.59 51.3) (width 0.5) (layer "B.Cu") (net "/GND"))
 (segment (start 114.75 65.75) (end 121.25 65.75) (width 0.5) (layer "B.Cu") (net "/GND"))
 (segment (start 90.75 65.75) (end 97.25 65.75) (width 0.5) (layer "B.Cu") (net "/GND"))
 (segment (start 201.78 53.975) (end 200.54 52.735) (width 0.5) (layer "B.Cu") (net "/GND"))
 (segment (start 201.85 63.47) (end 201.85 56.83) (width 0.5) (layer "B.Cu") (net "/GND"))
 (segment (start 197.43 67.89) (end 201.85 63.47) (width 0.5) (layer "B.Cu") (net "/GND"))
 (segment (start 169.25 65.75) (end 170.83 65.75) (width 0.5) (layer "B.Cu") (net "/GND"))
 (segment (start 160.31 68.19) (end 162.75 65.75) (width 0.5) (layer "B.Cu") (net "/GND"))
 (segment (start 170.83 65.75) (end 172.97 67.89) (width 0.5) (layer "B.Cu") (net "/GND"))
 (segment (start 143.59 51.3) (end 138.89 56) (width 0.5) (layer "B.Cu") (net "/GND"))
 (segment (start 201.78 54.36) (end 201.78 53.975) (width 0.5) (layer "B.Cu") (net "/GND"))
 (segment (start 121.25 65.75) (end 123.67 68.17) (width 0.5) (layer "B.Cu") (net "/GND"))
 (segment (start 200.54 52.735) (end 199.105 51.3) (width 0.5) (layer "B.Cu") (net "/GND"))
 (segment (start 136.35 54.62) (end 136.35 56) (width 0.2) (layer "F.Cu") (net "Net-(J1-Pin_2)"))
 (segment (start 203.08 55.275) (end 199.645 58.71) (width 0.2) (layer "F.Cu") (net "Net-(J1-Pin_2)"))
 (segment (start 199.645 58.71) (end 186.05 58.71) (width 0.2) (layer "F.Cu") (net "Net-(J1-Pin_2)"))
 (segment (start 186.05 58.71) (end 181.08 53.74) (width 0.2) (layer "F.Cu") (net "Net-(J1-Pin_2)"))
 (segment (start 137.23 53.74) (end 136.35 54.62) (width 0.2) (layer "F.Cu") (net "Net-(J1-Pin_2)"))
 (segment (start 181.08 53.74) (end 137.23 53.74) (width 0.2) (layer "F.Cu") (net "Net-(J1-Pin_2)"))
 (segment (start 201.095 50.75) (end 139.06 50.75) (width 0.2) (layer "B.Cu") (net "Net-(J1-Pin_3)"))
 (segment (start 203.08 52.735) (end 201.095 50.75) (width 0.2) (layer "B.Cu") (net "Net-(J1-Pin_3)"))
 (segment (start 139.06 50.75) (end 133.81 56) (width 0.2) (layer "B.Cu") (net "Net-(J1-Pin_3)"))
 (segment (start 131.27 56) (end 131.27 56.54) (width 0.2) (layer "F.Cu") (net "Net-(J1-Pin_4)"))
 (segment (start 201.725 59.17) (end 205.62 55.275) (width 0.2) (layer "F.Cu") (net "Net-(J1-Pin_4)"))
 (segment (start 185.43 59.17) (end 201.725 59.17) (width 0.2) (layer "F.Cu") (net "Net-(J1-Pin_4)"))
 (segment (start 183.8 57.54) (end 185.43 59.17) (width 0.2) (layer "F.Cu") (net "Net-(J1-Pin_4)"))
 (segment (start 132.27 57.54) (end 183.8 57.54) (width 0.2) (layer "F.Cu") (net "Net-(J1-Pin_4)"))
 (segment (start 131.27 56.54) (end 132.27 57.54) (width 0.2) (layer "F.Cu") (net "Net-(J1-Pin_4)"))
 (segment (start 205.62 52.735) (end 204.253077 51.368077) (width 0.2) (layer "F.Cu") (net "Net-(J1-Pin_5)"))
 (segment (start 204.253077 51.368077) (end 133.361923 51.368077) (width 0.2) (layer "F.Cu") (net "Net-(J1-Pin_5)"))
 (segment (start 133.361923 51.368077) (end 128.73 56) (width 0.2) (layer "F.Cu") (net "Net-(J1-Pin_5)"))
 (segment (start 203.715 59.72) (end 184.9 59.72) (width 0.2) (layer "F.Cu") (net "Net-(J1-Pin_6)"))
 (segment (start 128.35 58.16) (end 126.19 56) (width 0.2) (layer "F.Cu") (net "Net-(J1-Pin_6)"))
 (segment (start 183.34 58.16) (end 128.35 58.16) (width 0.2) (layer "F.Cu") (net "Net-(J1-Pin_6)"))
 (segment (start 208.16 55.275) (end 203.715 59.72) (width 0.2) (layer "F.Cu") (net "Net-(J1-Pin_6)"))
 (segment (start 184.9 59.72) (end 183.34 58.16) (width 0.2) (layer "F.Cu") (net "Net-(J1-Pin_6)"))
 (segment (start 127.09 50.74) (end 123.65 54.18) (width 0.2) (layer "F.Cu") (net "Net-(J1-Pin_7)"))
 (segment (start 208.16 52.735) (end 206.165 50.74) (width 0.2) (layer "F.Cu") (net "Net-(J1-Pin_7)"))
 (segment (start 206.165 50.74) (end 127.09 50.74) (width 0.2) (layer "F.Cu") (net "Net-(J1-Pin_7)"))
 (segment (start 123.65 54.18) (end 123.65 56) (width 0.2) (layer "F.Cu") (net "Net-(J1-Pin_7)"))
 (segment (start 123.97 58.86) (end 121.11 56) (width 0.2) (layer "F.Cu") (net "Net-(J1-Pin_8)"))
 (segment (start 210.7 55.275) (end 205.055 60.92) (width 0.2) (layer "F.Cu") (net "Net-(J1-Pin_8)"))
 (segment (start 182.99 58.86) (end 123.97 58.86) (width 0.2) (layer "F.Cu") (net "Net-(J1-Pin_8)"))
 (segment (start 205.055 60.92) (end 185.05 60.92) (width 0.2) (layer "F.Cu") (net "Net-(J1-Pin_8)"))
 (segment (start 185.05 60.92) (end 182.99 58.86) (width 0.2) (layer "F.Cu") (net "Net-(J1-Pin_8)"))
 (segment (start 171.754 63.754) (end 173.3065 63.754) (width 0.25) (layer "B.Cu") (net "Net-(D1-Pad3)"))
 (segment (start 162.75 61.25) (end 169.25 61.25) (width 0.25) (layer "B.Cu") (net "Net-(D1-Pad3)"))
 (segment (start 169.25 61.25) (end 171.754 63.754) (width 0.25) (layer "B.Cu") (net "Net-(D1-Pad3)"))
 (segment (start 114.75 61.25) (end 121.25 61.25) (width 0.25) (layer "B.Cu") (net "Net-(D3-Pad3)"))
 (segment (start 121.25 61.25) (end 123.754 63.754) (width 0.25) (layer "B.Cu") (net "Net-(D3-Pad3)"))
 (segment (start 123.754 63.754) (end 125.5545 63.754) (width 0.25) (layer "B.Cu") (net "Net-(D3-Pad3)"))
 (segment (start 147.754 63.754) (end 149.4305 63.754) (width 0.25) (layer "B.Cu") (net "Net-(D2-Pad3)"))
 (segment (start 138.75 61.25) (end 145.25 61.25) (width 0.25) (layer "B.Cu") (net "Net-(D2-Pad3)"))
 (segment (start 145.25 61.25) (end 147.754 63.754) (width 0.25) (layer "B.Cu") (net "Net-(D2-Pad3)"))
 (segment (start 103.4565 65.532) (end 102.122 65.532) (width 0.25) (layer "B.Cu") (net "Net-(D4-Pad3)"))
 (segment (start 100.87 64.28) (end 100.87 61.25) (width 0.25) (layer "B.Cu") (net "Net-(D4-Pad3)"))
 (segment (start 90.75 61.25) (end 97.25 61.25) (width 0.25) (layer "B.Cu") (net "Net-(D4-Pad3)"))
 (segment (start 97.25 61.25) (end 100.87 61.25) (width 0.25) (layer "B.Cu") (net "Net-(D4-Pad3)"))
 (segment (start 101.16 60.96) (end 103.4565 60.96) (width 0.25) (layer "B.Cu") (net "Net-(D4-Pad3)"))
 (segment (start 100.87 61.25) (end 101.16 60.96) (width 0.25) (layer "B.Cu") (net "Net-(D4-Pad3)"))
 (segment (start 102.122 65.532) (end 100.87 64.28) (width 0.25) (layer "B.Cu") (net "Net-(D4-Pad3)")))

